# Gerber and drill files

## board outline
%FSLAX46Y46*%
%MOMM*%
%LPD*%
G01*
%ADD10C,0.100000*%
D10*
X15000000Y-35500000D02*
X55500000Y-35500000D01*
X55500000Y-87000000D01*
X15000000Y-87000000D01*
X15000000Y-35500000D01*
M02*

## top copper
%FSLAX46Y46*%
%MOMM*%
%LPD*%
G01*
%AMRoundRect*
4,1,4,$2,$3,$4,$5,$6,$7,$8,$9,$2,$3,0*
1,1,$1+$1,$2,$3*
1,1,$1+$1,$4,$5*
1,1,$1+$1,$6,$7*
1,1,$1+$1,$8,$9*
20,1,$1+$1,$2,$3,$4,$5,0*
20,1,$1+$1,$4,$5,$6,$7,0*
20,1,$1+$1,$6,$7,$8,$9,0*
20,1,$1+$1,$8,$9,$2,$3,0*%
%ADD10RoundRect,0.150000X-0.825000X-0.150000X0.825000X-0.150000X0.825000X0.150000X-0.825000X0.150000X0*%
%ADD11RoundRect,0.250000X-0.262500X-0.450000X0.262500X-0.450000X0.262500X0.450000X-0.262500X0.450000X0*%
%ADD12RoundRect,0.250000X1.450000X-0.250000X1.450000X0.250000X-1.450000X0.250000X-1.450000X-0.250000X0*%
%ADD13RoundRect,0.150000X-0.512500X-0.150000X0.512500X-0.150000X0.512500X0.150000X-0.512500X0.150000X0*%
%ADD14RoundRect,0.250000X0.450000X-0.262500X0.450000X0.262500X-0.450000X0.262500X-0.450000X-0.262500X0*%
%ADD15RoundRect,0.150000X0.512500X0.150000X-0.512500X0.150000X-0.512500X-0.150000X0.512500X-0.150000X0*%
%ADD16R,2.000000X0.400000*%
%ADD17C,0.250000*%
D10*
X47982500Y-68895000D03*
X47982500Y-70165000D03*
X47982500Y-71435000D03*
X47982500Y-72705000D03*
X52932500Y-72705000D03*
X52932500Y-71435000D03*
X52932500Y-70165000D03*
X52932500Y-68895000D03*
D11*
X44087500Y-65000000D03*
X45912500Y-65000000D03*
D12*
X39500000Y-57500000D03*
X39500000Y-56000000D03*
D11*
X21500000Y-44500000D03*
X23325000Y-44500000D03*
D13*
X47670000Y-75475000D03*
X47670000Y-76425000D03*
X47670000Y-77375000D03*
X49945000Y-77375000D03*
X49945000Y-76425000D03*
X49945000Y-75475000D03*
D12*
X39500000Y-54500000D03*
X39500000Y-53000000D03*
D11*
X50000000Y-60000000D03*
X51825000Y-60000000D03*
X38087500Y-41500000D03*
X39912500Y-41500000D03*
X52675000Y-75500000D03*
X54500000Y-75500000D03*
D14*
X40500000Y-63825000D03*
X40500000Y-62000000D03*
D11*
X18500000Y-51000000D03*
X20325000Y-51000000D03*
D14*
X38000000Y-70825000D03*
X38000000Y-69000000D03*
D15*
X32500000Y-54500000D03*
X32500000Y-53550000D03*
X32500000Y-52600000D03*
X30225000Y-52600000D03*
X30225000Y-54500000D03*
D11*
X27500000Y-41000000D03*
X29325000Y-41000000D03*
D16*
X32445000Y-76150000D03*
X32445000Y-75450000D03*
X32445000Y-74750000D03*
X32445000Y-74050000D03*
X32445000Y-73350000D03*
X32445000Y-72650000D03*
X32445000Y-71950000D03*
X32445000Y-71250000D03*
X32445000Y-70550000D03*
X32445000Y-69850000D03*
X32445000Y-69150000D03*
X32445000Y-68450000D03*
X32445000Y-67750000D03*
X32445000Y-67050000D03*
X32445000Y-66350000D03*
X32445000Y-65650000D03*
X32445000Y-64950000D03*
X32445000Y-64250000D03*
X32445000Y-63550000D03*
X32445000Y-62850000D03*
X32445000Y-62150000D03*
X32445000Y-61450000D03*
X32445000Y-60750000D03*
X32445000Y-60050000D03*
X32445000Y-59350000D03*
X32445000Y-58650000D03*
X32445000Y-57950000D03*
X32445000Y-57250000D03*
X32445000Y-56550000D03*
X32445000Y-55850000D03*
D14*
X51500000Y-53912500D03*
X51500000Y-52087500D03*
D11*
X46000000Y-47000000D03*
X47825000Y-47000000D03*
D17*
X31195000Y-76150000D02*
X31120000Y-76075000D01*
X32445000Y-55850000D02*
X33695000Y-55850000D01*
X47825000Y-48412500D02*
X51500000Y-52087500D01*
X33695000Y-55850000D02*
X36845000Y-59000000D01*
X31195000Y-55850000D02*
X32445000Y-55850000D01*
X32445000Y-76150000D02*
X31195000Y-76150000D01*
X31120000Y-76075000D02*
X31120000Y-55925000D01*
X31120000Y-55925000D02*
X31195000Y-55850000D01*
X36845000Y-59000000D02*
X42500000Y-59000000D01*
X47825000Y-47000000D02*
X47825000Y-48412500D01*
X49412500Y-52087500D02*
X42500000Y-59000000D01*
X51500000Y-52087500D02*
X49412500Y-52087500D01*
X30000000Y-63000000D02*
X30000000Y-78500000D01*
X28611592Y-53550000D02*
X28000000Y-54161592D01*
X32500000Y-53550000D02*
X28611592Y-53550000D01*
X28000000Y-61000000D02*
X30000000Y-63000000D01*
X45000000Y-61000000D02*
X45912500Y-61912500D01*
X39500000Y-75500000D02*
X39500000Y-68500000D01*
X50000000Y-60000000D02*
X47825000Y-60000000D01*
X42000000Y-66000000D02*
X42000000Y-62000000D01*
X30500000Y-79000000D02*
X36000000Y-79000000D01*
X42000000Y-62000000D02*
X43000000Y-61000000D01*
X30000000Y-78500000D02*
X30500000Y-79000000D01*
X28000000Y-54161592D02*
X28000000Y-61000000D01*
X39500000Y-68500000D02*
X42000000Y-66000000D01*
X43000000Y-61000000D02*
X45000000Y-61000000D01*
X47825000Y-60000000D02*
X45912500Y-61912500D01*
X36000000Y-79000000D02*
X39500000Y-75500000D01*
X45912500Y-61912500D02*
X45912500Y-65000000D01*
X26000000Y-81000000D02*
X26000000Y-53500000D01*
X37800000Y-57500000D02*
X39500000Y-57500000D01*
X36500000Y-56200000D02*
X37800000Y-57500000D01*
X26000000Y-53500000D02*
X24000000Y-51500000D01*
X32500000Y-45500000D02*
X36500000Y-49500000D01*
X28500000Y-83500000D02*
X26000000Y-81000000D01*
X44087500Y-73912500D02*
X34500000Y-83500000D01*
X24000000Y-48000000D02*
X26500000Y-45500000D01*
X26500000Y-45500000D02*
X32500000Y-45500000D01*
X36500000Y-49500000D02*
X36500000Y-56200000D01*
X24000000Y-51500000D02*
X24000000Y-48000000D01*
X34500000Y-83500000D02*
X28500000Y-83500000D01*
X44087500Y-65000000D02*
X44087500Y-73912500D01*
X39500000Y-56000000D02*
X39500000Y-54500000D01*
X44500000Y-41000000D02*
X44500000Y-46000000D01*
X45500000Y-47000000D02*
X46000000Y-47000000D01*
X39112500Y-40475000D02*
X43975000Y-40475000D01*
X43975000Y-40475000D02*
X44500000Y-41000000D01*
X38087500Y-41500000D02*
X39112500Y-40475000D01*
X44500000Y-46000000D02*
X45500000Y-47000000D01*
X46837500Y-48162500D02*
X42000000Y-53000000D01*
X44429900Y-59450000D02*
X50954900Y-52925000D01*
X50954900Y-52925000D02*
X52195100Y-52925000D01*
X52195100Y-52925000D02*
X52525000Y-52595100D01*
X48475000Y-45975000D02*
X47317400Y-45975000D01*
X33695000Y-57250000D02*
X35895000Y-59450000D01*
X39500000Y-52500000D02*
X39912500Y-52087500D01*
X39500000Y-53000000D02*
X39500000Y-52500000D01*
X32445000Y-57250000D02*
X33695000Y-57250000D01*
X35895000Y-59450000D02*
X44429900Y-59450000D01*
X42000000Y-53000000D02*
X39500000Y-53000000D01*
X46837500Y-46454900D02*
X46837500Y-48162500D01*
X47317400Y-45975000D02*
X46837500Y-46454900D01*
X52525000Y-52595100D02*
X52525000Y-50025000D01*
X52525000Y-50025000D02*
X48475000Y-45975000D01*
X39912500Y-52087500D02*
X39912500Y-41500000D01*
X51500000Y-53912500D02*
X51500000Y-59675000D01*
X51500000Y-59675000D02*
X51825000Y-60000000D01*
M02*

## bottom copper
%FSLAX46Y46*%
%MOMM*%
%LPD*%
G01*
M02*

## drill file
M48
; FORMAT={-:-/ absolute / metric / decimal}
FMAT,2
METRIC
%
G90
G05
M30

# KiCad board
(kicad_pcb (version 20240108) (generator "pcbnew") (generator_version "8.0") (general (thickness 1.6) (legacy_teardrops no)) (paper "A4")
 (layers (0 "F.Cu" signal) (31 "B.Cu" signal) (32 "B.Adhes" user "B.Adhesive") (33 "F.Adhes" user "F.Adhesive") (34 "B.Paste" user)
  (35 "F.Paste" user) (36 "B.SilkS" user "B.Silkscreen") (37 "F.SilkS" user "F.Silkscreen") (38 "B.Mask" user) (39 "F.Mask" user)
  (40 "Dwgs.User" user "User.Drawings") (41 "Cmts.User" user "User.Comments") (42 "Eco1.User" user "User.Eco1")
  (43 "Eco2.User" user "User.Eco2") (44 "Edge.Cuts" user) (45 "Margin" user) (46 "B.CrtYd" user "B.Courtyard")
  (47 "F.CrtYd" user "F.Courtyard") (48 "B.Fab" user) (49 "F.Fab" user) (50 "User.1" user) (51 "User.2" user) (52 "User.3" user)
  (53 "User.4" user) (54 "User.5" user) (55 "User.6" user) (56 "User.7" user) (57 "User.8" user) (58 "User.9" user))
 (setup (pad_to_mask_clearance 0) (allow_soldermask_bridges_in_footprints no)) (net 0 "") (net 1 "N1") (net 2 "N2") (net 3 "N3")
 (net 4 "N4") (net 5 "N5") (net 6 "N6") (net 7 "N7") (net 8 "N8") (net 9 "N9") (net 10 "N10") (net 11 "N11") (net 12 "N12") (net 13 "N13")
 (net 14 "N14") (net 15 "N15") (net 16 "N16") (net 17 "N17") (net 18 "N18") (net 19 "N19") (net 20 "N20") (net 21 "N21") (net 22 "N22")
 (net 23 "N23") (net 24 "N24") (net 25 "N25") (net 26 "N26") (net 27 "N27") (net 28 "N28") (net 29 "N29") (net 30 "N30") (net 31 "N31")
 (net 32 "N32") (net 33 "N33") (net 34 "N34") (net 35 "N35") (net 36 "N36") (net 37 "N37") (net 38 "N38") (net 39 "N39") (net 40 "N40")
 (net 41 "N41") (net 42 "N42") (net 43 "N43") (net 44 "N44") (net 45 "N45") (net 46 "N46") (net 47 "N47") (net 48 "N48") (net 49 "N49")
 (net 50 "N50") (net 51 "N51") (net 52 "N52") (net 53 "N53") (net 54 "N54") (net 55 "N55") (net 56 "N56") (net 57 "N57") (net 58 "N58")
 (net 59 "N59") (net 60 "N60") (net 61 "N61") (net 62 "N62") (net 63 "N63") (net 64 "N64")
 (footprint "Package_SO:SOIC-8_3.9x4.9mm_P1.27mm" (layer "F.Cu") (at 50.4575 70.8)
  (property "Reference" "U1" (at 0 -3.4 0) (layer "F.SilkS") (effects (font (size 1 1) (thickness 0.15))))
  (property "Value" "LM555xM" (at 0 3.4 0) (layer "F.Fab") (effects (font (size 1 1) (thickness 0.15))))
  (pad "1" smd roundrect (at -2.475 -1.905) (size 1.95 0.6) (layers "F.Cu" "F.Paste" "F.Mask") (roundrect_rratio 0.25) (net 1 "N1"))
  (pad "2" smd roundrect (at -2.475 -0.635) (size 1.95 0.6) (layers "F.Cu" "F.Paste" "F.Mask") (roundrect_rratio 0.25) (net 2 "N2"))
  (pad "3" smd roundrect (at -2.475 0.635) (size 1.95 0.6) (layers "F.Cu" "F.Paste" "F.Mask") (roundrect_rratio 0.25) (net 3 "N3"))
  (pad "4" smd roundrect (at -2.475 1.905) (size 1.95 0.6) (layers "F.Cu" "F.Paste" "F.Mask") (roundrect_rratio 0.25) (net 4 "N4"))
  (pad "5" smd roundrect (at 2.475 1.905) (size 1.95 0.6) (layers "F.Cu" "F.Paste" "F.Mask") (roundrect_rratio 0.25) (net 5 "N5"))
  (pad "6" smd roundrect (at 2.475 0.635) (size 1.95 0.6) (layers "F.Cu" "F.Paste" "F.Mask") (roundrect_rratio 0.25) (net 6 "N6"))
  (pad "7" smd roundrect (at 2.475 -0.635) (size 1.95 0.6) (layers "F.Cu" "F.Paste" "F.Mask") (roundrect_rratio 0.25) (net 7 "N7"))
  (pad "8" smd roundrect (at 2.475 -1.905) (size 1.95 0.6) (layers "F.Cu" "F.Paste" "F.Mask") (roundrect_rratio 0.25) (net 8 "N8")))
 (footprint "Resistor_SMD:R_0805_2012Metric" (layer "F.Cu") (at 45 65)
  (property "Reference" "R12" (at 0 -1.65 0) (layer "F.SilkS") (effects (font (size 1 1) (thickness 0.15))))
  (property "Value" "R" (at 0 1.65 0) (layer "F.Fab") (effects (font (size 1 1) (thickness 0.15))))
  (pad "1" smd roundrect (at -0.9125 0) (size 1.025 1.4) (layers "F.Cu" "F.Paste" "F.Mask") (roundrect_rratio 0.243902) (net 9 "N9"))
  (pad "2" smd roundrect (at 0.9125 0) (size 1.025 1.4) (layers "F.Cu" "F.Paste" "F.Mask") (roundrect_rratio 0.243902) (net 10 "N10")))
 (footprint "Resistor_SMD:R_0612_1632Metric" (layer "F.Cu") (at 39.5 56.75 90)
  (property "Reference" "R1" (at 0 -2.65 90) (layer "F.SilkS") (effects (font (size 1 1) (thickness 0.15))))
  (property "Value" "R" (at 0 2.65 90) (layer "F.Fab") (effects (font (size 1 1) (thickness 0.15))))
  (pad "1" smd roundrect (at -0.75 0 90) (size 1 3.4) (layers "F.Cu" "F.Paste" "F.Mask") (roundrect_rratio 0.25) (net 9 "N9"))
  (pad "2" smd roundrect (at 0.75 0 90) (size 1 3.4) (layers "F.Cu" "F.Paste" "F.Mask") (roundrect_rratio 0.25) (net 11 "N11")))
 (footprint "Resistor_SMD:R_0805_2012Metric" (layer "F.Cu") (at 22.4125 44.5)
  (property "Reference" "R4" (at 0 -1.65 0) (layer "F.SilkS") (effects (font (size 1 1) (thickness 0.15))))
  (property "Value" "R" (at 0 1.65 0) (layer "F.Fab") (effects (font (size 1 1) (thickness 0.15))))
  (pad "1" smd roundrect (at -0.9125 0) (size 1.025 1.4) (layers "F.Cu" "F.Paste" "F.Mask") (roundrect_rratio 0.243902) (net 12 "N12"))
  (pad "2" smd roundrect (at 0.9125 0) (size 1.025 1.4) (layers "F.Cu" "F.Paste" "F.Mask") (roundrect_rratio 0.243902) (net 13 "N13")))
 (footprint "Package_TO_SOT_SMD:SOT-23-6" (layer "F.Cu") (at 48.8075 76.425)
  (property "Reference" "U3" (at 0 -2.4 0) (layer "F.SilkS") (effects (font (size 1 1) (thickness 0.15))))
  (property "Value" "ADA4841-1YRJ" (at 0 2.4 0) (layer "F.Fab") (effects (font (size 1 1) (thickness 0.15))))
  (pad "1" smd roundrect (at -1.1375 -0.95) (size 1.325 0.6) (layers "F.Cu" "F.Paste" "F.Mask") (roundrect_rratio 0.25) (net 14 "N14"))
  (pad "2" smd roundrect (at -1.1375 0) (size 1.325 0.6) (layers "F.Cu" "F.Paste" "F.Mask") (roundrect_rratio 0.25) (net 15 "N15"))
  (pad "3" smd roundrect (at -1.1375 0.95) (size 1.325 0.6) (layers "F.Cu" "F.Paste" "F.Mask") (roundrect_rratio 0.25) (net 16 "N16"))
  (pad "4" smd roundrect (at 1.1375 0.95) (size 1.325 0.6) (layers "F.Cu" "F.Paste" "F.Mask") (roundrect_rratio 0.25) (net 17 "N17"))
  (pad "5" smd roundrect (at 1.1375 0) (size 1.325 0.6) (layers "F.Cu" "F.Paste" "F.Mask") (roundrect_rratio 0.25) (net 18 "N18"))
  (pad "6" smd roundrect (at 1.1375 -0.95) (size 1.325 0.6) (layers "F.Cu" "F.Paste" "F.Mask") (roundrect_rratio 0.25) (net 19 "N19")))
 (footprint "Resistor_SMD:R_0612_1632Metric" (layer "F.Cu") (at 39.5 53.75 90)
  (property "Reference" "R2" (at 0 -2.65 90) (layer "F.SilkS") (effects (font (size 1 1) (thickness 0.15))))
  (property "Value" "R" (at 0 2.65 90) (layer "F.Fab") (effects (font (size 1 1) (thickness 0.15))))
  (pad "1" smd roundrect (at -0.75 0 90) (size 1 3.4) (layers "F.Cu" "F.Paste" "F.Mask") (roundrect_rratio 0.25) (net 11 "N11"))
  (pad "2" smd roundrect (at 0.75 0 90) (size 1 3.4) (layers "F.Cu" "F.Paste" "F.Mask") (roundrect_rratio 0.25) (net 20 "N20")))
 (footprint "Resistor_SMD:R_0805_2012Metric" (layer "F.Cu") (at 50.9125 60)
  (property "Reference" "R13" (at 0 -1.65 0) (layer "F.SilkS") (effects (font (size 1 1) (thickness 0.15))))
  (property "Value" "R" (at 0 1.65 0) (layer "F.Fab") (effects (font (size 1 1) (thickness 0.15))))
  (pad "1" smd roundrect (at -0.9125 0) (size 1.025 1.4) (layers "F.Cu" "F.Paste" "F.Mask") (roundrect_rratio 0.243902) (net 10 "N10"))
  (pad "2" smd roundrect (at 0.9125 0) (size 1.025 1.4) (layers "F.Cu" "F.Paste" "F.Mask") (roundrect_rratio 0.243902) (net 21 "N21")))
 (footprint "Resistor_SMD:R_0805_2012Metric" (layer "F.Cu") (at 39 41.5)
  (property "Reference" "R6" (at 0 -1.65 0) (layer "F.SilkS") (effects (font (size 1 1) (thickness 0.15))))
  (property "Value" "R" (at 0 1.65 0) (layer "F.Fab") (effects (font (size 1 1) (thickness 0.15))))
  (pad "1" smd roundrect (at -0.9125 0) (size 1.025 1.4) (layers "F.Cu" "F.Paste" "F.Mask") (roundrect_rratio 0.243902) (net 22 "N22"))
  (pad "2" smd roundrect (at 0.9125 0) (size 1.025 1.4) (layers "F.Cu" "F.Paste" "F.Mask") (roundrect_rratio 0.243902) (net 20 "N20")))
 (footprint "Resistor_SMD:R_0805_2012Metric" (layer "F.Cu") (at 53.5875 75.5)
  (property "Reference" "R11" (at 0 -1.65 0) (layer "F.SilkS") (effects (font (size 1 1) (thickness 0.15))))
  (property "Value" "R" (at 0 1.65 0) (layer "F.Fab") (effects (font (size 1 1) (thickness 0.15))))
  (pad "1" smd roundrect (at -0.9125 0) (size 1.025 1.4) (layers "F.Cu" "F.Paste" "F.Mask") (roundrect_rratio 0.243902) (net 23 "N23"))
  (pad "2" smd roundrect (at 0.9125 0) (size 1.025 1.4) (layers "F.Cu" "F.Paste" "F.Mask") (roundrect_rratio 0.243902) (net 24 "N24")))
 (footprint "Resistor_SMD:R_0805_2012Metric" (layer "F.Cu") (at 40.5 62.9125 90)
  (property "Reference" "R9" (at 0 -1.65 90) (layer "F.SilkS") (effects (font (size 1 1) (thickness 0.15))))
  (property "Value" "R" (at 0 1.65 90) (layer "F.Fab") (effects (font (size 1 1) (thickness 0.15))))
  (pad "1" smd roundrect (at -0.9125 0 90) (size 1.025 1.4) (layers "F.Cu" "F.Paste" "F.Mask") (roundrect_rratio 0.243902) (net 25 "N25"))
  (pad "2" smd roundrect (at 0.9125 0 90) (size 1.025 1.4) (layers "F.Cu" "F.Paste" "F.Mask") (roundrect_rratio 0.243902) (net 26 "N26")))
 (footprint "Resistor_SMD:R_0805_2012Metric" (layer "F.Cu") (at 19.4125 51)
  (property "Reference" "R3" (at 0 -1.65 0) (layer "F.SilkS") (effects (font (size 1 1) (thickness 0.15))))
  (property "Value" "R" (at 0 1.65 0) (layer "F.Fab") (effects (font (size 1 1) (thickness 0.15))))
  (pad "1" smd roundrect (at -0.9125 0) (size 1.025 1.4) (layers "F.Cu" "F.Paste" "F.Mask") (roundrect_rratio 0.243902) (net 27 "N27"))
  (pad "2" smd roundrect (at 0.9125 0) (size 1.025 1.4) (layers "F.Cu" "F.Paste" "F.Mask") (roundrect_rratio 0.243902) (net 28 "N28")))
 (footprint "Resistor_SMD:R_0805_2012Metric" (layer "F.Cu") (at 38 69.9125 90)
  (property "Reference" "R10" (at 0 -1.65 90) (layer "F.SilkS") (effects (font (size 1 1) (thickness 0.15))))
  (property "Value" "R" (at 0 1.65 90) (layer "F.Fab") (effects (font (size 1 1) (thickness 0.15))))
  (pad "1" smd roundrect (at -0.9125 0 90) (size 1.025 1.4) (layers "F.Cu" "F.Paste" "F.Mask") (roundrect_rratio 0.243902) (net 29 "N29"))
  (pad "2" smd roundrect (at 0.9125 0 90) (size 1.025 1.4) (layers "F.Cu" "F.Paste" "F.Mask") (roundrect_rratio 0.243902) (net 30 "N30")))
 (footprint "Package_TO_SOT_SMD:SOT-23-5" (layer "F.Cu") (at 31.3625 53.55 180)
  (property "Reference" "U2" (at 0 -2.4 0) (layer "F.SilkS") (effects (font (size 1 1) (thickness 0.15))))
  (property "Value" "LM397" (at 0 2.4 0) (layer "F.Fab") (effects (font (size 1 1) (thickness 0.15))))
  (pad "1" smd roundrect (at -1.1375 -0.95 180) (size 1.325 0.6) (layers "F.Cu" "F.Paste" "F.Mask") (roundrect_rratio 0.25) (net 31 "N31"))
  (pad "2" smd roundrect (at -1.1375 0 180) (size 1.325 0.6) (layers "F.Cu" "F.Paste" "F.Mask") (roundrect_rratio 0.25) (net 10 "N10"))
  (pad "3" smd roundrect (at -1.1375 0.95 180) (size 1.325 0.6) (layers "F.Cu" "F.Paste" "F.Mask") (roundrect_rratio 0.25) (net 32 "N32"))
  (pad "4" smd roundrect (at 1.1375 0.95 180) (size 1.325 0.6) (layers "F.Cu" "F.Paste" "F.Mask") (roundrect_rratio 0.25) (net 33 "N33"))
  (pad "5" smd roundrect (at 1.1375 -0.95 180) (size 1.325 0.6) (layers "F.Cu" "F.Paste" "F.Mask") (roundrect_rratio 0.25) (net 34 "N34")))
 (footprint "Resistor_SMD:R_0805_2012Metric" (layer "F.Cu") (at 28.4125 41)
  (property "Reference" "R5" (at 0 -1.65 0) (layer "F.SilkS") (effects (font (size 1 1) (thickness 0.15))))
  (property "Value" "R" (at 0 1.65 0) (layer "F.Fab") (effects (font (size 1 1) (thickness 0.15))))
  (pad "1" smd roundrect (at -0.9125 0) (size 1.025 1.4) (layers "F.Cu" "F.Paste" "F.Mask") (roundrect_rratio 0.243902) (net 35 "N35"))
  (pad "2" smd roundrect (at 0.9125 0) (size 1.025 1.4) (layers "F.Cu" "F.Paste" "F.Mask") (roundrect_rratio 0.243902) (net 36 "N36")))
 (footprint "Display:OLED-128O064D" (layer "F.Cu") (at 32.445 66 90)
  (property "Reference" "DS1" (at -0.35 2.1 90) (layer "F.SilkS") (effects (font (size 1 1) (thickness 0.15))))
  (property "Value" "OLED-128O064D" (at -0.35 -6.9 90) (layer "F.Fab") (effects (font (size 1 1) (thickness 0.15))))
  (pad "1" smd rect (at -10.15 0 90) (size 0.4 2) (layers "F.Cu" "F.Paste" "F.Mask") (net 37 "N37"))
  (pad "2" smd rect (at -9.45 0 90) (size 0.4 2) (layers "F.Cu" "F.Paste" "F.Mask") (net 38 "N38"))
  (pad "3" smd rect (at -8.75 0 90) (size 0.4 2) (layers "F.Cu" "F.Paste" "F.Mask") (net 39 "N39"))
  (pad "4" smd rect (at -8.05 0 90) (size 0.4 2) (layers "F.Cu" "F.Paste" "F.Mask") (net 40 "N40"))
  (pad "5" smd rect (at -7.35 0 90) (size 0.4 2) (layers "F.Cu" "F.Paste" "F.Mask") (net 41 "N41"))
  (pad "6" smd rect (at -6.65 0 90) (size 0.4 2) (layers "F.Cu" "F.Paste" "F.Mask") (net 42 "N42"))
  (pad "7" smd rect (at -5.95 0 90) (size 0.4 2) (layers "F.Cu" "F.Paste" "F.Mask") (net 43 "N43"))
  (pad "8" smd rect (at -5.25 0 90) (size 0.4 2) (layers "F.Cu" "F.Paste" "F.Mask") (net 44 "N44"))
  (pad "9" smd rect (at -4.55 0 90) (size 0.4 2) (layers "F.Cu" "F.Paste" "F.Mask") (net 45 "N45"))
  (pad "10" smd rect (at -3.85 0 90) (size 0.4 2) (layers "F.Cu" "F.Paste" "F.Mask") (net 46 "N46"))
  (pad "11" smd rect (at -3.15 0 90) (size 0.4 2) (layers "F.Cu" "F.Paste" "F.Mask") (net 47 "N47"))
  (pad "12" smd rect (at -2.45 0 90) (size 0.4 2) (layers "F.Cu" "F.Paste" "F.Mask") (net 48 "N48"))
  (pad "13" smd rect (at -1.75 0 90) (size 0.4 2) (layers "F.Cu" "F.Paste" "F.Mask") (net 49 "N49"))
  (pad "14" smd rect (at -1.05 0 90) (size 0.4 2) (layers "F.Cu" "F.Paste" "F.Mask") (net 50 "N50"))
  (pad "15" smd rect (at -0.35 0 90) (size 0.4 2) (layers "F.Cu" "F.Paste" "F.Mask") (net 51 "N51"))
  (pad "16" smd rect (at 0.35 0 90) (size 0.4 2) (layers "F.Cu" "F.Paste" "F.Mask") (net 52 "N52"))
  (pad "17" smd rect (at 1.05 0 90) (size 0.4 2) (layers "F.Cu" "F.Paste" "F.Mask") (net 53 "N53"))
  (pad "18" smd rect (at 1.75 0 90) (size 0.4 2) (layers "F.Cu" "F.Paste" "F.Mask") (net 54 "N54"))
  (pad "19" smd rect (at 2.45 0 90) (size 0.4 2) (layers "F.Cu" "F.Paste" "F.Mask") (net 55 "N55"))
  (pad "20" smd rect (at 3.15 0 90) (size 0.4 2) (layers "F.Cu" "F.Paste" "F.Mask") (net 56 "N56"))
  (pad "21" smd rect (at 3.85 0 90) (size 0.4 2) (layers "F.Cu" "F.Paste" "F.Mask") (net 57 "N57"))
  (pad "22" smd rect (at 4.55 0 90) (size 0.4 2) (layers "F.Cu" "F.Paste" "F.Mask") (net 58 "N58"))
  (pad "23" smd rect (at 5.25 0 90) (size 0.4 2) (layers "F.Cu" "F.Paste" "F.Mask") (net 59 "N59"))
  (pad "24" smd rect (at 5.95 0 90) (size 0.4 2) (layers "F.Cu" "F.Paste" "F.Mask") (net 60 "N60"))
  (pad "25" smd rect (at 6.65 0 90) (size 0.4 2) (layers "F.Cu" "F.Paste" "F.Mask") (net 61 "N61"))
  (pad "26" smd rect (at 7.35 0 90) (size 0.4 2) (layers "F.Cu" "F.Paste" "F.Mask") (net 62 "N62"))
  (pad "27" smd rect (at 8.05 0 90) (size 0.4 2) (layers "F.Cu" "F.Paste" "F.Mask") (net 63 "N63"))
  (pad "28" smd rect (at 8.75 0 90) (size 0.4 2) (layers "F.Cu" "F.Paste" "F.Mask") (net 20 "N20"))
  (pad "29" smd rect (at 9.45 0 90) (size 0.4 2) (layers "F.Cu" "F.Paste" "F.Mask") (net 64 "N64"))
  (pad "30" smd rect (at 10.15 0 90) (size 0.4 2) (layers "F.Cu" "F.Paste" "F.Mask") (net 37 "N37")))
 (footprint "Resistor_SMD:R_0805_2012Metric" (layer "F.Cu") (at 51.5 53 90)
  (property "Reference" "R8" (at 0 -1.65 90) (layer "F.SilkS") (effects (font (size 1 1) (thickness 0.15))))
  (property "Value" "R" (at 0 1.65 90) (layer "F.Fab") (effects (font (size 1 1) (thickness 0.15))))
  (pad "1" smd roundrect (at -0.9125 0 90) (size 1.025 1.4) (layers "F.Cu" "F.Paste" "F.Mask") (roundrect_rratio 0.243902) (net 21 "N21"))
  (pad "2" smd roundrect (at 0.9125 0 90) (size 1.025 1.4) (layers "F.Cu" "F.Paste" "F.Mask") (roundrect_rratio 0.243902) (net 37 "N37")))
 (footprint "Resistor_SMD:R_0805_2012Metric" (layer "F.Cu") (at 46.9125 47)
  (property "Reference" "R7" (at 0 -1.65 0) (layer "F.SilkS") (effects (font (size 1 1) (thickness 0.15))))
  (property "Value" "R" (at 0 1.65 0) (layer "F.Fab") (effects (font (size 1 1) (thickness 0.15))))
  (pad "1" smd roundrect (at -0.9125 0) (size 1.025 1.4) (layers "F.Cu" "F.Paste" "F.Mask") (roundrect_rratio 0.243902) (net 22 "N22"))
  (pad "2" smd roundrect (at 0.9125 0) (size 1.025 1.4) (layers "F.Cu" "F.Paste" "F.Mask") (roundrect_rratio 0.243902) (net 37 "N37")))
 (gr_rect (start 15 35.5) (end 55.5 87) (stroke (width 0.1) (type default)) (fill none) (layer "Edge.Cuts"))
 (segment (start 31.195 76.15) (end 31.12 76.075) (width 0.25) (layer "F.Cu") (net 37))
 (segment (start 32.445 55.85) (end 33.695 55.85) (width 0.25) (layer "F.Cu") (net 37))
 (segment (start 47.825 48.4125) (end 51.5 52.0875) (width 0.25) (layer "F.Cu") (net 37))
 (segment (start 33.695 55.85) (end 36.845 59) (width 0.25) (layer "F.Cu") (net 37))
 (segment (start 31.195 55.85) (end 32.445 55.85) (width 0.25) (layer "F.Cu") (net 37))
 (segment (start 32.445 76.15) (end 31.195 76.15) (width 0.25) (layer "F.Cu") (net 37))
 (segment (start 31.12 76.075) (end 31.12 55.925) (width 0.25) (layer "F.Cu") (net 37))
 (segment (start 31.12 55.925) (end 31.195 55.85) (width 0.25) (layer "F.Cu") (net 37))
 (segment (start 36.845 59) (end 42.5 59) (width 0.25) (layer "F.Cu") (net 37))
 (segment (start 47.825 47) (end 47.825 48.4125) (width 0.25) (layer "F.Cu") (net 37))
 (segment (start 49.4125 52.0875) (end 42.5 59) (width 0.25) (layer "F.Cu") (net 37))
 (segment (start 51.5 52.0875) (end 49.4125 52.0875) (width 0.25) (layer "F.Cu") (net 37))
 (segment (start 30 63) (end 30 78.5) (width 0.25) (layer "F.Cu") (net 10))
 (segment (start 28.611592 53.55) (end 28 54.161592) (width 0.25) (layer "F.Cu") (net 10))
 (segment (start 32.5 53.55) (end 28.611592 53.55) (width 0.25) (layer "F.Cu") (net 10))
 (segment (start 28 61) (end 30 63) (width 0.25) (layer "F.Cu") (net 10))
 (segment (start 45 61) (end 45.9125 61.9125) (width 0.25) (layer "F.Cu") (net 10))
 (segment (start 39.5 75.5) (end 39.5 68.5) (width 0.25) (layer "F.Cu") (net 10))
 (segment (start 50 60) (end 47.825 60) (width 0.25) (layer "F.Cu") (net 10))
 (segment (start 42 66) (end 42 62) (width 0.25) (layer "F.Cu") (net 10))
 (segment (start 30.5 79) (end 36 79) (width 0.25) (layer "F.Cu") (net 10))
 (segment (start 42 62) (end 43 61) (width 0.25) (layer "F.Cu") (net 10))
 (segment (start 30 78.5) (end 30.5 79) (width 0.25) (layer "F.Cu") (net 10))
 (segment (start 28 54.161592) (end 28 61) (width 0.25) (layer "F.Cu") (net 10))
 (segment (start 39.5 68.5) (end 42 66) (width 0.25) (layer "F.Cu") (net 10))
 (segment (start 43 61) (end 45 61) (width 0.25) (layer "F.Cu") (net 10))
 (segment (start 47.825 60) (end 45.9125 61.9125) (width 0.25) (layer "F.Cu") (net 10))
 (segment (start 36 79) (end 39.5 75.5) (width 0.25) (layer "F.Cu") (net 10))
 (segment (start 45.9125 61.9125) (end 45.9125 65) (width 0.25) (layer "F.Cu") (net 10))
 (segment (start 26 81) (end 26 53.5) (width 0.25) (layer "F.Cu") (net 9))
 (segment (start 37.8 57.5) (end 39.5 57.5) (width 0.25) (layer "F.Cu") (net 9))
 (segment (start 36.5 56.2) (end 37.8 57.5) (width 0.25) (layer "F.Cu") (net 9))
 (segment (start 26 53.5) (end 24 51.5) (width 0.25) (layer "F.Cu") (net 9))
 (segment (start 32.5 45.5) (end 36.5 49.5) (width 0.25) (layer "F.Cu") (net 9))
 (segment (start 28.5 83.5) (end 26 81) (width 0.25) (layer "F.Cu") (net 9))
 (segment (start 44.0875 73.9125) (end 34.5 83.5) (width 0.25) (layer "F.Cu") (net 9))
 (segment (start 24 48) (end 26.5 45.5) (width 0.25) (layer "F.Cu") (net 9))
 (segment (start 26.5 45.5) (end 32.5 45.5) (width 0.25) (layer "F.Cu") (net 9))
 (segment (start 36.5 49.5) (end 36.5 56.2) (width 0.25) (layer "F.Cu") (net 9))
 (segment (start 24 51.5) (end 24 48) (width 0.25) (layer "F.Cu") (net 9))
 (segment (start 34.5 83.5) (end 28.5 83.5) (width 0.25) (layer "F.Cu") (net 9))
 (segment (start 44.0875 65) (end 44.0875 73.9125) (width 0.25) (layer "F.Cu") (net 9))
 (segment (start 39.5 56) (end 39.5 54.5) (width 0.25) (layer "F.Cu") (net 11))
 (segment (start 44.5 41) (end 44.5 46) (width 0.25) (layer "F.Cu") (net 22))
 (segment (start 45.5 47) (end 46 47) (width 0.25) (layer "F.Cu") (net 22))
 (segment (start 39.1125 40.475) (end 43.975 40.475) (width 0.25) (layer "F.Cu") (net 22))
 (segment (start 43.975 40.475) (end 44.5 41) (width 0.25) (layer "F.Cu") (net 22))
 (segment (start 38.0875 41.5) (end 39.1125 40.475) (width 0.25) (layer "F.Cu") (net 22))
 (segment (start 44.5 46) (end 45.5 47) (width 0.25) (layer "F.Cu") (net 22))
 (segment (start 46.8375 48.1625) (end 42 53) (width 0.25) (layer "F.Cu") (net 20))
 (segment (start 44.4299 59.45) (end 50.9549 52.925) (width 0.25) (layer "F.Cu") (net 20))
 (segment (start 50.9549 52.925) (end 52.1951 52.925) (width 0.25) (layer "F.Cu") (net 20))
 (segment (start 52.1951 52.925) (end 52.525 52.5951) (width 0.25) (layer "F.Cu") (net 20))
 (segment (start 48.475 45.975) (end 47.3174 45.975) (width 0.25) (layer "F.Cu") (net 20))
 (segment (start 33.695 57.25) (end 35.895 59.45) (width 0.25) (layer "F.Cu") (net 20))
 (segment (start 39.5 52.5) (end 39.9125 52.0875) (width 0.25) (layer "F.Cu") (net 20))
 (segment (start 39.5 53) (end 39.5 52.5) (width 0.25) (layer "F.Cu") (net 20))
 (segment (start 32.445 57.25) (end 33.695 57.25) (width 0.25) (layer "F.Cu") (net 20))
 (segment (start 35.895 59.45) (end 44.4299 59.45) (width 0.25) (layer "F.Cu") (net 20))
 (segment (start 42 53) (end 39.5 53) (width 0.25) (layer "F.Cu") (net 20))
 (segment (start 46.8375 46.4549) (end 46.8375 48.1625) (width 0.25) (layer "F.Cu") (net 20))
 (segment (start 47.3174 45.975) (end 46.8375 46.4549) (width 0.25) (layer "F.Cu") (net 20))
 (segment (start 52.525 52.5951) (end 52.525 50.025) (width 0.25) (layer "F.Cu") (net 20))
 (segment (start 52.525 50.025) (end 48.475 45.975) (width 0.25) (layer "F.Cu") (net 20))
 (segment (start 39.9125 52.0875) (end 39.9125 41.5) (width 0.25) (layer "F.Cu") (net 20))
 (segment (start 51.5 53.9125) (end 51.5 59.675) (width 0.25) (layer "F.Cu") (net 21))
 (segment (start 51.5 59.675) (end 51.825 60) (width 0.25) (layer "F.Cu") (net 21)))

